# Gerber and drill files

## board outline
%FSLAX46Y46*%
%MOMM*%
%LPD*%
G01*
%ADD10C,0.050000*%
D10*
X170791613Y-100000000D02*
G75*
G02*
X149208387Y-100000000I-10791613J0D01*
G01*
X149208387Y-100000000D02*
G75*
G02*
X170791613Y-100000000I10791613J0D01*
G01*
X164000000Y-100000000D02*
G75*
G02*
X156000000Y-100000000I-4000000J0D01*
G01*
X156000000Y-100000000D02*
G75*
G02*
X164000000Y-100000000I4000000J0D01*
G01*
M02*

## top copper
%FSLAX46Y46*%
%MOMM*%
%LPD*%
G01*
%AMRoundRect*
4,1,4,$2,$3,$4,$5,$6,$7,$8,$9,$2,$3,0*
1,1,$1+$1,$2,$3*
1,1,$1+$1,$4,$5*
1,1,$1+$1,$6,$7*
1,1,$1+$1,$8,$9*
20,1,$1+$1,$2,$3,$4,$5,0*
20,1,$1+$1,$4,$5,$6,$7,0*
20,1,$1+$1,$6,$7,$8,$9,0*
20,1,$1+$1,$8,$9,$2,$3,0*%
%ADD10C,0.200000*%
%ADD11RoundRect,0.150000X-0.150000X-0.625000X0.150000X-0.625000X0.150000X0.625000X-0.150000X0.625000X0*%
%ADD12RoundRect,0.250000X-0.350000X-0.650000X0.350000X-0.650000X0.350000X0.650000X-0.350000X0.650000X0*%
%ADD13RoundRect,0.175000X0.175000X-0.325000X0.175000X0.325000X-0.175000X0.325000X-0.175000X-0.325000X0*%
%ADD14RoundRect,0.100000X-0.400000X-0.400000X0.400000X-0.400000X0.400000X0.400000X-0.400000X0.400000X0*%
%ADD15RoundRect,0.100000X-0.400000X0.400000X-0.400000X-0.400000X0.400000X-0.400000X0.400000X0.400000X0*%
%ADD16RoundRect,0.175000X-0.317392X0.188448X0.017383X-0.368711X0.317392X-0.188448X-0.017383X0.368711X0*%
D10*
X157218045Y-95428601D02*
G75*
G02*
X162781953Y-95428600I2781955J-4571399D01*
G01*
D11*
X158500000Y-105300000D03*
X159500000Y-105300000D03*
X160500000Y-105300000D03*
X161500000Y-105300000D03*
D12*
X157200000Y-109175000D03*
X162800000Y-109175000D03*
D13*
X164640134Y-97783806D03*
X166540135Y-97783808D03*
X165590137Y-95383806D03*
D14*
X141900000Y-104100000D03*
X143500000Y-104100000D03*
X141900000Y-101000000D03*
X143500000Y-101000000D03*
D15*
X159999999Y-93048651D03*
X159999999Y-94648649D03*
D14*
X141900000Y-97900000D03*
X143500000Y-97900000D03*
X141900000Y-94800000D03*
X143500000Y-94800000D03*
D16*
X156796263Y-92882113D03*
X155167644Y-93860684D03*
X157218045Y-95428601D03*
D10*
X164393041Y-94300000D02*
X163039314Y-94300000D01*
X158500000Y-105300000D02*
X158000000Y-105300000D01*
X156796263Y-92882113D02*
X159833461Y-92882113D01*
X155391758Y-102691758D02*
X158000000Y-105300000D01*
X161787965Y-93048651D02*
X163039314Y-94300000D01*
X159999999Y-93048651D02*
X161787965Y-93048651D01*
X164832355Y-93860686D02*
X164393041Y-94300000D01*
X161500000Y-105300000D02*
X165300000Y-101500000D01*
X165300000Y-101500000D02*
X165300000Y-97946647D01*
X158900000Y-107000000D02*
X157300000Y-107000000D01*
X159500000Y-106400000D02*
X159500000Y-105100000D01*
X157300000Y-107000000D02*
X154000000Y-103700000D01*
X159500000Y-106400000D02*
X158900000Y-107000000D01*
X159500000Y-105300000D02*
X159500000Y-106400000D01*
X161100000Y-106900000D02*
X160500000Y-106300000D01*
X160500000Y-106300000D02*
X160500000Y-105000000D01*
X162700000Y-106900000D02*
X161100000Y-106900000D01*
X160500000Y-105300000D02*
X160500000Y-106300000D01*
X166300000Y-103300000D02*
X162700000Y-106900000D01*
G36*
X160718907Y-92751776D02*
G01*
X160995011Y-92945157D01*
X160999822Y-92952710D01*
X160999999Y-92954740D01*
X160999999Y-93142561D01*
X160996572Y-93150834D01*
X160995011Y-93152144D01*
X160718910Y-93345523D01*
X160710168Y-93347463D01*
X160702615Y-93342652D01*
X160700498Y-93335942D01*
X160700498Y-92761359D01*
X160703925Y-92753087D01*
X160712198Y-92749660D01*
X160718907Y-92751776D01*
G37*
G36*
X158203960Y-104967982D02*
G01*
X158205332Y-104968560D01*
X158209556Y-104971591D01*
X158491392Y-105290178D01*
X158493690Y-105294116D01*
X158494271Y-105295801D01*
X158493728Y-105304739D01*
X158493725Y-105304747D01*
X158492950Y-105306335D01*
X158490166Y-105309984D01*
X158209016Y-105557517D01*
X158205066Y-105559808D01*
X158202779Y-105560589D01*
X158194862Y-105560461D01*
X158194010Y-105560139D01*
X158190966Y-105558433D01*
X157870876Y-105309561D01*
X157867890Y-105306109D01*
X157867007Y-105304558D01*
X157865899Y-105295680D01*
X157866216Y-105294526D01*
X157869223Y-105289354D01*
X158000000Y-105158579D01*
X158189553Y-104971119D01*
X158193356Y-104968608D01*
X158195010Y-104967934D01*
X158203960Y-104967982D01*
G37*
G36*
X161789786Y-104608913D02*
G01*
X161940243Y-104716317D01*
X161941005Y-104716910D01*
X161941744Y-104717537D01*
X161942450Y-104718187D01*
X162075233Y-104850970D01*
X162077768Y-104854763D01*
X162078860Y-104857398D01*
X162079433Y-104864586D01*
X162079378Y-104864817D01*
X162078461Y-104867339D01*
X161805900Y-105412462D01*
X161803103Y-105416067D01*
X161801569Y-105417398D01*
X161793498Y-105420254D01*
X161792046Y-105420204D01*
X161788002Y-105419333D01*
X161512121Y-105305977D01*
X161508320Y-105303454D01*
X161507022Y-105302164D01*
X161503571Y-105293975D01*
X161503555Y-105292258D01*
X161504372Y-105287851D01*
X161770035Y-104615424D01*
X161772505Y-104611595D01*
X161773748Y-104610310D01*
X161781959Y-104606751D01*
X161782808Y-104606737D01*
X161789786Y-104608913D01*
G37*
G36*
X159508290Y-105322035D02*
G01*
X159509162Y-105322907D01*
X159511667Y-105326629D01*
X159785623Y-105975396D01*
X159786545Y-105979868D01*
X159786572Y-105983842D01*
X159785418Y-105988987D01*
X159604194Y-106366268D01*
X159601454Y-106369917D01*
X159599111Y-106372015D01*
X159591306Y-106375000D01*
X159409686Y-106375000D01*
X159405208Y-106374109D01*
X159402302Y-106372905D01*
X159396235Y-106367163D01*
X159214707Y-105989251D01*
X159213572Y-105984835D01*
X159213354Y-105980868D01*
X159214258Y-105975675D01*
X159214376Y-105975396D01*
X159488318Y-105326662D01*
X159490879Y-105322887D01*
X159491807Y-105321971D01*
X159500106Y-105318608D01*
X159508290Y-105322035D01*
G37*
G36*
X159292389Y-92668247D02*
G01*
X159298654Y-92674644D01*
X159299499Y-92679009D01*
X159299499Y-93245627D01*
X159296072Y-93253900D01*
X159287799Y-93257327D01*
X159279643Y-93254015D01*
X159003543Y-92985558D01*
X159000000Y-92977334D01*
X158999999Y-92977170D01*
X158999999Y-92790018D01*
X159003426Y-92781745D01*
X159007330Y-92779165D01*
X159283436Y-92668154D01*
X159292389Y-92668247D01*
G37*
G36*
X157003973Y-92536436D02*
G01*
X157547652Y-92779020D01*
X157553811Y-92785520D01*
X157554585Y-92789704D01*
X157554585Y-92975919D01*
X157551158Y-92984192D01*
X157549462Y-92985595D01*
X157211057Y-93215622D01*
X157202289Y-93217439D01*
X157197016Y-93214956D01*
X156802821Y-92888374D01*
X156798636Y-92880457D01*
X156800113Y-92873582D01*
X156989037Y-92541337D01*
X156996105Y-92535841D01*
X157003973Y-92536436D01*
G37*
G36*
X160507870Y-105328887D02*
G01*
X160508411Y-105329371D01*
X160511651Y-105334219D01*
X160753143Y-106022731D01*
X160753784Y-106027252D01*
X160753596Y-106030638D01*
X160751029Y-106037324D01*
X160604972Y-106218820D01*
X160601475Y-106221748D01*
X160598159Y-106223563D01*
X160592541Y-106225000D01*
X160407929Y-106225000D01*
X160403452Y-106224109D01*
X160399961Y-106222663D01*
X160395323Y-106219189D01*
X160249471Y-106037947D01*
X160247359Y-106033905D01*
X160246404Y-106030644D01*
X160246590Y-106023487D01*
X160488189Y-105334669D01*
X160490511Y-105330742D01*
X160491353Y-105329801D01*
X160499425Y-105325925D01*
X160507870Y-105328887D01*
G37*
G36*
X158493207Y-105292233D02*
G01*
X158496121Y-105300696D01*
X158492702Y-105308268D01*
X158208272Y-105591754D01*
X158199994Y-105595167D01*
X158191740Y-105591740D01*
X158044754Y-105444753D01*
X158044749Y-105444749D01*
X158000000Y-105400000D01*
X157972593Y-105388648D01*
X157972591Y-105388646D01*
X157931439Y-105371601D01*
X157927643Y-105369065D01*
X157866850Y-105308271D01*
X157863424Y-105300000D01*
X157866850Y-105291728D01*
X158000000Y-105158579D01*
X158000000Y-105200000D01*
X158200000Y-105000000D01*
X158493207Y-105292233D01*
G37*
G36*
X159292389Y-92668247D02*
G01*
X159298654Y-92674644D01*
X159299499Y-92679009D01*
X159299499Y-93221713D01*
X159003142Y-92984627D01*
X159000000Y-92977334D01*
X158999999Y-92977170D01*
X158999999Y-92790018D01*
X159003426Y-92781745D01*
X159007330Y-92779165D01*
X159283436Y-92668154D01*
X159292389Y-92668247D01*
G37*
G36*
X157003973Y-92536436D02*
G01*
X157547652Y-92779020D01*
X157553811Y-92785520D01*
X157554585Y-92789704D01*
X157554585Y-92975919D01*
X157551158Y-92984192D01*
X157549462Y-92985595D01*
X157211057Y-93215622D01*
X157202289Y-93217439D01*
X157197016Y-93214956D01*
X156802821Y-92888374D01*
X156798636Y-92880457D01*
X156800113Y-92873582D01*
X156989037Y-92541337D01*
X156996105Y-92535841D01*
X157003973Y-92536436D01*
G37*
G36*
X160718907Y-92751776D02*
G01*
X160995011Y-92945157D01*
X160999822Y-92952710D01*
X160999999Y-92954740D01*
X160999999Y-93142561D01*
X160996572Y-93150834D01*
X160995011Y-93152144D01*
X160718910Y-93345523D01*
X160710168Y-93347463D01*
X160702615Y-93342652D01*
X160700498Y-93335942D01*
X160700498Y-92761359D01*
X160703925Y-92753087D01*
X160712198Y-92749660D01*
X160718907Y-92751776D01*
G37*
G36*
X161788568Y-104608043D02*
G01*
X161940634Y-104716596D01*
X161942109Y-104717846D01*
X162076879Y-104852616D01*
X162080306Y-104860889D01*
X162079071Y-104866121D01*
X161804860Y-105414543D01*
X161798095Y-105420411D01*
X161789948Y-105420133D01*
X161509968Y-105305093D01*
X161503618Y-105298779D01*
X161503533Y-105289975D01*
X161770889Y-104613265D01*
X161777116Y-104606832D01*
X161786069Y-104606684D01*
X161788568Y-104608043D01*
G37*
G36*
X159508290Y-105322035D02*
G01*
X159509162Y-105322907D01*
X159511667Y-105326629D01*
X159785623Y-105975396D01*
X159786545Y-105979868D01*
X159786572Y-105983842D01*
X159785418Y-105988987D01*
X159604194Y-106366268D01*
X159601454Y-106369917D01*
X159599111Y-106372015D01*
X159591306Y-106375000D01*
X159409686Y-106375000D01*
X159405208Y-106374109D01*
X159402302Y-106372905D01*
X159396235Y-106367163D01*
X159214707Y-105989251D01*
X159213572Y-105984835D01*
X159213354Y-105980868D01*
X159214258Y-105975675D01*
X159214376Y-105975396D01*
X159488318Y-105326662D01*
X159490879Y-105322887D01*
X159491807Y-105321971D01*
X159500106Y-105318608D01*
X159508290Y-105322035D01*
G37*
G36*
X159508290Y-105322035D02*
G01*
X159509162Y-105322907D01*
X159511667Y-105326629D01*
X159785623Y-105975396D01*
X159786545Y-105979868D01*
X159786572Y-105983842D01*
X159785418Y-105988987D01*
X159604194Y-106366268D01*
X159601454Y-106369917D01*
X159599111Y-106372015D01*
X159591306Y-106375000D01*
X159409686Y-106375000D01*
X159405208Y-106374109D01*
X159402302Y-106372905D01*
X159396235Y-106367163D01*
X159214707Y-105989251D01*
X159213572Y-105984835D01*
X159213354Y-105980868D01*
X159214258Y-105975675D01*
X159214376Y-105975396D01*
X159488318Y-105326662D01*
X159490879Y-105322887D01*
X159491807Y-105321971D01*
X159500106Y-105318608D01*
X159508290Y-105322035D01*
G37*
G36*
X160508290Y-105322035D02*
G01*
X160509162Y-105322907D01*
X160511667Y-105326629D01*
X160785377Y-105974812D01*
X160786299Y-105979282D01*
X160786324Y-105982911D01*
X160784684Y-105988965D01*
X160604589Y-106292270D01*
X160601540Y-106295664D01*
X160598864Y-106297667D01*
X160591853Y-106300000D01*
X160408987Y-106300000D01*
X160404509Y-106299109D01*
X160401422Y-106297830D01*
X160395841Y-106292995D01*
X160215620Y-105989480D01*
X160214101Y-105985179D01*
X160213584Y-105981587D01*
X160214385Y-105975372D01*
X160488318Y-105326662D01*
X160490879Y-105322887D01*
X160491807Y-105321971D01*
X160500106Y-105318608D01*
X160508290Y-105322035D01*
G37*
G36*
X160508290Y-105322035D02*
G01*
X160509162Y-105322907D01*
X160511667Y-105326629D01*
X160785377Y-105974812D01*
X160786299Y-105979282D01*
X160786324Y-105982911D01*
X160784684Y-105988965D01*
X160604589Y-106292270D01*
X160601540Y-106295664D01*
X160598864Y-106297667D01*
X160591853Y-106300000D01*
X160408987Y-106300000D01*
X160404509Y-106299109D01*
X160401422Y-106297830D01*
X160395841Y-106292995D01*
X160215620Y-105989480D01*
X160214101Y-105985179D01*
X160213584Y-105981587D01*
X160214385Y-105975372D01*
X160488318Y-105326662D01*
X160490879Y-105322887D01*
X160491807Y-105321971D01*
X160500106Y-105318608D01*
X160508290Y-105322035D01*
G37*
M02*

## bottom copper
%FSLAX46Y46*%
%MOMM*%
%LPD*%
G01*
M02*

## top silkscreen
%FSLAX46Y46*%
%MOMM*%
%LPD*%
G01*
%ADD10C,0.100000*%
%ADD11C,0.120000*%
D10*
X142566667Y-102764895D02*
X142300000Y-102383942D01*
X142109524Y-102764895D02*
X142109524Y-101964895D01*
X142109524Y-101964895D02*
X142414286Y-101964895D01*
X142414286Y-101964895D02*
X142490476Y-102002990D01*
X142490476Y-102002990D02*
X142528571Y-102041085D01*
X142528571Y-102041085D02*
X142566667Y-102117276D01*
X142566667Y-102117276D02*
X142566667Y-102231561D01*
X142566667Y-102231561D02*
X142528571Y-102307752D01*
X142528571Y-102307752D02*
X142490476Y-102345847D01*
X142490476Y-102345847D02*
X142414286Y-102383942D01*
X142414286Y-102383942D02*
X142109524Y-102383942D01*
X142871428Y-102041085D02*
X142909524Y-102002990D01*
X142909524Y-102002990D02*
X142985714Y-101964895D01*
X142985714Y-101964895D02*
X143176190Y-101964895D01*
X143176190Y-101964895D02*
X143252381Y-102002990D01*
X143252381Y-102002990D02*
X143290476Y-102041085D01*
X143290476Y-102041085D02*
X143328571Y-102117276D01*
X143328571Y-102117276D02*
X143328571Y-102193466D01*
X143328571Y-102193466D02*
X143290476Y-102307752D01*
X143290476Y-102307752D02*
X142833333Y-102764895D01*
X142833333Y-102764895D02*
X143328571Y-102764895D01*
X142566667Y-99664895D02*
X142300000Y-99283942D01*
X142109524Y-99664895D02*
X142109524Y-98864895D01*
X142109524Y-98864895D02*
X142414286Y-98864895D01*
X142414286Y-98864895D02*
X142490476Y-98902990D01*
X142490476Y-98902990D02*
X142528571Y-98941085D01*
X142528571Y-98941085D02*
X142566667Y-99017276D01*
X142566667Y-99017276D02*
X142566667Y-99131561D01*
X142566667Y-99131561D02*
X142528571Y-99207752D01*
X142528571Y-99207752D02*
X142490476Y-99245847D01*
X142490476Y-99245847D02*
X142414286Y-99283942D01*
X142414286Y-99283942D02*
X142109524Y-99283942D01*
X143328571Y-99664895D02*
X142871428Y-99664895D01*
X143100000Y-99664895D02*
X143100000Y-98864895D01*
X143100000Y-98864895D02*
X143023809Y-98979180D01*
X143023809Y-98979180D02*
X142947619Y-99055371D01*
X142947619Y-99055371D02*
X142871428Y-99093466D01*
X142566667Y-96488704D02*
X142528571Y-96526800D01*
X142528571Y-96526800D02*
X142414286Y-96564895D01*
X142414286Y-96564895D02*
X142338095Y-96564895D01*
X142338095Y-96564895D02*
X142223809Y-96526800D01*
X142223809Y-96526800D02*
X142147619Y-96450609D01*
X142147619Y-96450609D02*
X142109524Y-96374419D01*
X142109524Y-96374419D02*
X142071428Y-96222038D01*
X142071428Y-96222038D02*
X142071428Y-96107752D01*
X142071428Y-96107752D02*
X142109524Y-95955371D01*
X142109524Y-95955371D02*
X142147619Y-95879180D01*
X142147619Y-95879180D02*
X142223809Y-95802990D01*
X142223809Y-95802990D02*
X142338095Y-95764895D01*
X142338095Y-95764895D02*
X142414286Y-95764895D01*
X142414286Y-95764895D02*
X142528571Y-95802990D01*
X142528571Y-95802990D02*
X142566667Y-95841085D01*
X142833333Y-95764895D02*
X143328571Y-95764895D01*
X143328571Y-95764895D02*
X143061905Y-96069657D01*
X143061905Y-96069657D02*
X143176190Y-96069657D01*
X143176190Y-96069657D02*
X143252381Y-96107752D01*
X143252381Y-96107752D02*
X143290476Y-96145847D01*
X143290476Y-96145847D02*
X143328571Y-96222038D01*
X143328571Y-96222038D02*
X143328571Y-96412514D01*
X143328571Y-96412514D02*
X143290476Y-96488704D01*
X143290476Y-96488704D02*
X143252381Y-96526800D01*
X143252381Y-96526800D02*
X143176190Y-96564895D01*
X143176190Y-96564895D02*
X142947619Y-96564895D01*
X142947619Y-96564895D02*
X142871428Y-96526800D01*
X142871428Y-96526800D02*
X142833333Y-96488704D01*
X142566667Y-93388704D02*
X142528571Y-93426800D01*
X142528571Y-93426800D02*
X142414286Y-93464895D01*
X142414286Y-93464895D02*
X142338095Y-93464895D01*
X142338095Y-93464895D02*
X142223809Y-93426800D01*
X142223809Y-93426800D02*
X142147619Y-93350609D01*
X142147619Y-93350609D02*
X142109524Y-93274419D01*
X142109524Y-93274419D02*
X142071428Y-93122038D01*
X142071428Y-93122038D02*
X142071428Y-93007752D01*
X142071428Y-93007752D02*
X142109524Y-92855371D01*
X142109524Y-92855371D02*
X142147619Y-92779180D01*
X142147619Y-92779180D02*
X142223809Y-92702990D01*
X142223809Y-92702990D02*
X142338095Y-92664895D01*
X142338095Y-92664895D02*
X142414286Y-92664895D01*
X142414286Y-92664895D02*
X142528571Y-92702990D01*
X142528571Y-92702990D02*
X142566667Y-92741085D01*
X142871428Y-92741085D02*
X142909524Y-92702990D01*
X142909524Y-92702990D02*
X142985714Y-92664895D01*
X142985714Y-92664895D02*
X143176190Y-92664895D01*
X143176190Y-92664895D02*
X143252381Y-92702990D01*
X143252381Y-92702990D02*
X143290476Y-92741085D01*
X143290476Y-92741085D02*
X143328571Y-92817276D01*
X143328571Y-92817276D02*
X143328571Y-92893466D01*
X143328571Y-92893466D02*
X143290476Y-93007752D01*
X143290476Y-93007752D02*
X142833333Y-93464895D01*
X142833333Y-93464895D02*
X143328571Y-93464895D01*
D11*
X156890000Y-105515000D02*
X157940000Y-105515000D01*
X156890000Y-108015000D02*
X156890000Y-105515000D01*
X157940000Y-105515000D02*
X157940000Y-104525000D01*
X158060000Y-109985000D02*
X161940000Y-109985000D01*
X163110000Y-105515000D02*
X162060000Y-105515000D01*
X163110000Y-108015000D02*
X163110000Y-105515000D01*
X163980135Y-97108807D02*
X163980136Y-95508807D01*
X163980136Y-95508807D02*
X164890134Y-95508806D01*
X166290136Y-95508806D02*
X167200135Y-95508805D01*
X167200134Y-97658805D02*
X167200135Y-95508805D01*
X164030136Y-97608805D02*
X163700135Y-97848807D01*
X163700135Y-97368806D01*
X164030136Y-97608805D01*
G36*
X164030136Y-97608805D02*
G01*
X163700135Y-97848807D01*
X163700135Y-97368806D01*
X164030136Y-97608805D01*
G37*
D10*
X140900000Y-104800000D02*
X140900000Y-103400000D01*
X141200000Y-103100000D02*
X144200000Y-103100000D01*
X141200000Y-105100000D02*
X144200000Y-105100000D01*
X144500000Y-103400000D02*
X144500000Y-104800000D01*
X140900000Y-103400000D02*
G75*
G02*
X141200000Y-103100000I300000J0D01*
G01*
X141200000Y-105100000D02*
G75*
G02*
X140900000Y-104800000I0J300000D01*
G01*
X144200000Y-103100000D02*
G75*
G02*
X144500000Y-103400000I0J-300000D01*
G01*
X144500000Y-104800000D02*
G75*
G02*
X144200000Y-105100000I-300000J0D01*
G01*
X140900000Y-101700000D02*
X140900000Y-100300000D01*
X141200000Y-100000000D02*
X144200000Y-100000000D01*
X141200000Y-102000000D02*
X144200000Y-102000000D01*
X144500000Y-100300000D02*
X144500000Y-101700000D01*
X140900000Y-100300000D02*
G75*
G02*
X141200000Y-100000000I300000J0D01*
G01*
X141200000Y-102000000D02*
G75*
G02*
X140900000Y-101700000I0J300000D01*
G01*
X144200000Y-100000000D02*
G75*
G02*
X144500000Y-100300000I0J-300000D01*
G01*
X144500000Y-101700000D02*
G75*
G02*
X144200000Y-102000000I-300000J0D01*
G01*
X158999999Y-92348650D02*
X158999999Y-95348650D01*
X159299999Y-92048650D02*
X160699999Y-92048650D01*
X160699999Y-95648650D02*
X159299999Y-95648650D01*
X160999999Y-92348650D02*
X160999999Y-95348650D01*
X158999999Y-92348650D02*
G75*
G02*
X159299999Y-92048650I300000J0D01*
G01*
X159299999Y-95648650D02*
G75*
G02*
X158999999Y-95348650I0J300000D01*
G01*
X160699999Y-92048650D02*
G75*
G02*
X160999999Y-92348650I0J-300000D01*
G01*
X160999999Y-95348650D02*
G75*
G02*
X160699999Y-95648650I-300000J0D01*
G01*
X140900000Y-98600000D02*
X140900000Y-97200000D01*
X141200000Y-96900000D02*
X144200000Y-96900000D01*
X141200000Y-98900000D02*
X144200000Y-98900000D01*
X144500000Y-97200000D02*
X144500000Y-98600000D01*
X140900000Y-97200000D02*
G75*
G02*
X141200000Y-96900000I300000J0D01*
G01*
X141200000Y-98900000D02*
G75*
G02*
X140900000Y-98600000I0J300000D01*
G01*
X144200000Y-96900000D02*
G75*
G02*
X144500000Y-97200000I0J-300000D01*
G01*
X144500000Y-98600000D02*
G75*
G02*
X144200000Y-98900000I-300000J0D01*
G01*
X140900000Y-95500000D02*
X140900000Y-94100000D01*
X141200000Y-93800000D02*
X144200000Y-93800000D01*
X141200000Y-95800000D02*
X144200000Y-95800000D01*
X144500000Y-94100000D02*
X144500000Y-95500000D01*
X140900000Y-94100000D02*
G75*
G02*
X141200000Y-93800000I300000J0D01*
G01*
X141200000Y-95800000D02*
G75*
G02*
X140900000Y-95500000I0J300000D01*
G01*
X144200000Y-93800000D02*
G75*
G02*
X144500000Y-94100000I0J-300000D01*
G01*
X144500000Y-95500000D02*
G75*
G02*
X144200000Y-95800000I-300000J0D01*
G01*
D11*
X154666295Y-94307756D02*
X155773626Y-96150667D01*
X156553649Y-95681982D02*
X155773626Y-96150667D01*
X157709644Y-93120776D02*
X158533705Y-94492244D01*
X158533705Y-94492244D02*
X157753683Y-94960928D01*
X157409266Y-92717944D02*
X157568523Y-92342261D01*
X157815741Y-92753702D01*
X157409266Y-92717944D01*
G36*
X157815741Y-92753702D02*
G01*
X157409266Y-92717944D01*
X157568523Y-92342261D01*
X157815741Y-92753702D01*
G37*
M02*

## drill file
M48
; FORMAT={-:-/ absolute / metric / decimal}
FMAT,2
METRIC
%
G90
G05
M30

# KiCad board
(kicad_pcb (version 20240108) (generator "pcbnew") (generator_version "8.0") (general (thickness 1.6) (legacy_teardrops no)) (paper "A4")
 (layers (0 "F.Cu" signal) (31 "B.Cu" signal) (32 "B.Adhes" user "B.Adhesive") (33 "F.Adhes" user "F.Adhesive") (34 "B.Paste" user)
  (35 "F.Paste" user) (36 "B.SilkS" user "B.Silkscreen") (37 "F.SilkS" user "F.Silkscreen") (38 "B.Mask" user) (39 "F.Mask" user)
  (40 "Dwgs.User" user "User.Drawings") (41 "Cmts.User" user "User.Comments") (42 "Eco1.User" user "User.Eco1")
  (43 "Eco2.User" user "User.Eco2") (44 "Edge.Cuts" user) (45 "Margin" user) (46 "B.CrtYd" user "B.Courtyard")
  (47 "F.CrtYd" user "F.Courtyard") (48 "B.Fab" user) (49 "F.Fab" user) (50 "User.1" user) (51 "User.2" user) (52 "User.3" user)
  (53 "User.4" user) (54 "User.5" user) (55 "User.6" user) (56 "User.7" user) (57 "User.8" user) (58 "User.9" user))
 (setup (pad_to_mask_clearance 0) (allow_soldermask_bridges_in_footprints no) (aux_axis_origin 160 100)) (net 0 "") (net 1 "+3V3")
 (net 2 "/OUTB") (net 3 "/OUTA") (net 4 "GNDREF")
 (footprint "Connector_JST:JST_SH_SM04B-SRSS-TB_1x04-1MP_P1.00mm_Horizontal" (layer "F.Cu") (at 160 107.3)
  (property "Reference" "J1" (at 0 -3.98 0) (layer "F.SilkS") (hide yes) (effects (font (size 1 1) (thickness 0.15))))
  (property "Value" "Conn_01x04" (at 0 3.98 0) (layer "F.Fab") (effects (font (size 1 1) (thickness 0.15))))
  (fp_line (start -3.11 -1.785) (end -2.06 -1.785) (stroke (width 0.12) (type solid)) (layer "F.SilkS"))
  (fp_line (start -3.11 0.715) (end -3.11 -1.785) (stroke (width 0.12) (type solid)) (layer "F.SilkS"))
  (fp_line (start -2.06 -1.785) (end -2.06 -2.775) (stroke (width 0.12) (type solid)) (layer "F.SilkS"))
  (fp_line (start -1.94 2.685) (end 1.94 2.685) (stroke (width 0.12) (type solid)) (layer "F.SilkS"))
  (fp_line (start 3.11 -1.785) (end 2.06 -1.785) (stroke (width 0.12) (type solid)) (layer "F.SilkS"))
  (fp_line (start 3.11 0.715) (end 3.11 -1.785) (stroke (width 0.12) (type solid)) (layer "F.SilkS"))
  (pad "1" smd roundrect (at -1.5 -2) (size 0.6 1.55) (layers "F.Cu" "F.Paste" "F.Mask") (roundrect_rratio 0.25) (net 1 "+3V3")
   (teardrops (best_length_ratio 0.5) (max_length 1) (best_width_ratio 1) (max_width 2) (curve_points 0) (filter_ratio 0.9) (enabled yes)
    (allow_two_segments yes) (prefer_zone_connections yes)))
  (pad "2" smd roundrect (at -0.5 -2) (size 0.6 1.55) (layers "F.Cu" "F.Paste" "F.Mask") (roundrect_rratio 0.25) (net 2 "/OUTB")
   (teardrops (best_length_ratio 0.5) (max_length 1) (best_width_ratio 1) (max_width 2) (curve_points 0) (filter_ratio 0.9) (enabled yes)
    (allow_two_segments yes) (prefer_zone_connections yes)))
  (pad "3" smd roundrect (at 0.5 -2) (size 0.6 1.55) (layers "F.Cu" "F.Paste" "F.Mask") (roundrect_rratio 0.25) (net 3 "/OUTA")
   (teardrops (best_length_ratio 0.5) (max_length 1) (best_width_ratio 1) (max_width 2) (curve_points 0) (filter_ratio 0.9) (enabled yes)
    (allow_two_segments yes) (prefer_zone_connections yes)))
  (pad "4" smd roundrect (at 1.5 -2) (size 0.6 1.55) (layers "F.Cu" "F.Paste" "F.Mask") (roundrect_rratio 0.25) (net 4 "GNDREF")
   (teardrops (best_length_ratio 0.5) (max_length 1) (best_width_ratio 1) (max_width 2) (curve_points 0) (filter_ratio 0.9) (enabled yes)
    (allow_two_segments yes) (prefer_zone_connections yes)))
  (pad "MP" smd roundrect (at -2.8 1.875) (size 1.2 1.8) (layers "F.Cu" "F.Paste" "F.Mask") (roundrect_rratio 0.208333)
   (teardrops (best_length_ratio 0.5) (max_length 1) (best_width_ratio 1) (max_width 2) (curve_points 0) (filter_ratio 0.9) (enabled yes)
    (allow_two_segments yes) (prefer_zone_connections yes)))
  (pad "MP" smd roundrect (at 2.8 1.875) (size 1.2 1.8) (layers "F.Cu" "F.Paste" "F.Mask") (roundrect_rratio 0.208333)
   (teardrops (best_length_ratio 0.5) (max_length 1) (best_width_ratio 1) (max_width 2) (curve_points 0) (filter_ratio 0.9) (enabled yes)
    (allow_two_segments yes) (prefer_zone_connections yes))))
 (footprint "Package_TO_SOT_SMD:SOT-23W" (layer "F.Cu") (at 165.590135 96.583806 90)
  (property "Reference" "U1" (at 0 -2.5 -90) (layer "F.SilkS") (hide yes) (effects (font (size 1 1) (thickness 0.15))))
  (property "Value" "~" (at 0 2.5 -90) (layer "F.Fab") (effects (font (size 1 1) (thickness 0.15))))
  (fp_line (start -0.525001 -1.61) (end 1.074999 -1.609999) (stroke (width 0.12) (type solid)) (layer "F.SilkS"))
  (fp_line (start 1.074999 -1.609999) (end 1.075 -0.700001) (stroke (width 0.12) (type solid)) (layer "F.SilkS"))
  (fp_line (start 1.075 0.700001) (end 1.075001 1.61) (stroke (width 0.12) (type solid)) (layer "F.SilkS"))
  (fp_line (start -1.074999 1.609999) (end 1.075001 1.61) (stroke (width 0.12) (type solid)) (layer "F.SilkS"))
  (fp_poly
   (pts (xy -1.024999 -1.559999) (xy -1.265001 -1.89) (xy -0.785 -1.89) (xy -1.024999 -1.559999)) (stroke (width 0.12) (type solid))
   (fill solid) (layer "F.SilkS"))
  (pad "1" smd roundrect (at -1.2 -0.950001 90) (size 1 0.7) (layers "F.Cu" "F.Paste" "F.Mask") (roundrect_rratio 0.25) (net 1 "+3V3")
   (teardrops (best_length_ratio 0.5) (max_length 1) (best_width_ratio 1) (max_width 2) (curve_points 0) (filter_ratio 0.9) (enabled yes)
    (allow_two_segments yes) (prefer_zone_connections yes)))
  (pad "2" smd roundrect (at -1.200002 0.95 90) (size 1 0.7) (layers "F.Cu" "F.Paste" "F.Mask") (roundrect_rratio 0.25) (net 3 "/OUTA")
   (teardrops (best_length_ratio 0.5) (max_length 1) (best_width_ratio 1) (max_width 2) (curve_points 0) (filter_ratio 0.9) (enabled yes)
    (allow_two_segments yes) (prefer_zone_connections yes)))
  (pad "3" smd roundrect (at 1.2 0.000002 90) (size 1 0.7) (layers "F.Cu" "F.Paste" "F.Mask") (roundrect_rratio 0.25) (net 4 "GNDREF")
   (teardrops (best_length_ratio 0.5) (max_length 1) (best_width_ratio 1) (max_width 2) (curve_points 0) (filter_ratio 0.9) (enabled yes)
    (allow_two_segments yes) (prefer_zone_connections yes))))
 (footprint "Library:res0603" (layer "F.Cu") (at 142.7 104.1)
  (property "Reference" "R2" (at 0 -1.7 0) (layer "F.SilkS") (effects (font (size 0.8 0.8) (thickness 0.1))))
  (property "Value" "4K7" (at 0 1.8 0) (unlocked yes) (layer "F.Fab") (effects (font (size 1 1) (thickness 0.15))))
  (fp_line (start -1.8 0.7) (end -1.8 -0.7) (stroke (width 0.1) (type default)) (layer "F.SilkS"))
  (fp_line (start -1.5 -1) (end 1.5 -1) (stroke (width 0.1) (type default)) (layer "F.SilkS"))
  (fp_line (start -1.5 1) (end 1.5 1) (stroke (width 0.1) (type default)) (layer "F.SilkS"))
  (fp_line (start 1.8 -0.7) (end 1.8 0.7) (stroke (width 0.1) (type default)) (layer "F.SilkS"))
  (fp_arc (start -1.8 -0.7) (mid -1.712132 -0.912132) (end -1.5 -1) (stroke (width 0.1) (type default)) (layer "F.SilkS"))
  (fp_arc (start -1.5 1) (mid -1.712132 0.912132) (end -1.8 0.7) (stroke (width 0.1) (type default)) (layer "F.SilkS"))
  (fp_arc (start 1.5 -1) (mid 1.712132 -0.912132) (end 1.8 -0.7) (stroke (width 0.1) (type default)) (layer "F.SilkS"))
  (fp_arc (start 1.8 0.7) (mid 1.712132 0.912132) (end 1.5 1) (stroke (width 0.1) (type default)) (layer "F.SilkS"))
  (pad "1" smd roundrect (at -0.8 0) (size 1 1) (layers "F.Cu" "F.Paste" "F.Mask") (roundrect_rratio 0.1) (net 2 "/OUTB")
   (thermal_bridge_angle 45)
   (teardrops (best_length_ratio 0.5) (max_length 1) (best_width_ratio 1) (max_width 1) (curve_points 10) (filter_ratio 0.9) (enabled yes)
    (allow_two_segments yes) (prefer_zone_connections yes)))
  (pad "2" smd roundrect (at 0.8 0) (size 1 1) (layers "F.Cu" "F.Paste" "F.Mask") (roundrect_rratio 0.1) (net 4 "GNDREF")
   (thermal_bridge_angle 45)
   (teardrops (best_length_ratio 0.5) (max_length 1) (best_width_ratio 1) (max_width 1) (curve_points 10) (filter_ratio 0.9) (enabled yes)
    (allow_two_segments yes) (prefer_zone_connections yes))))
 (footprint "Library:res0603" (layer "F.Cu") (at 142.7 101)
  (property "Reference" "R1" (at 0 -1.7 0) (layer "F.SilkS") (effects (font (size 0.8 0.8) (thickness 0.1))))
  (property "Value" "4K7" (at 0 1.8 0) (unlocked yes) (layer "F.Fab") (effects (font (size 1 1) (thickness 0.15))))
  (fp_line (start -1.8 0.7) (end -1.8 -0.7) (stroke (width 0.1) (type default)) (layer "F.SilkS"))
  (fp_line (start -1.5 -1) (end 1.5 -1) (stroke (width 0.1) (type default)) (layer "F.SilkS"))
  (fp_line (start -1.5 1) (end 1.5 1) (stroke (width 0.1) (type default)) (layer "F.SilkS"))
  (fp_line (start 1.8 -0.7) (end 1.8 0.7) (stroke (width 0.1) (type default)) (layer "F.SilkS"))
  (fp_arc (start -1.8 -0.7) (mid -1.712132 -0.912132) (end -1.5 -1) (stroke (width 0.1) (type default)) (layer "F.SilkS"))
  (fp_arc (start -1.5 1) (mid -1.712132 0.912132) (end -1.8 0.7) (stroke (width 0.1) (type default)) (layer "F.SilkS"))
  (fp_arc (start 1.5 -1) (mid 1.712132 -0.912132) (end 1.8 -0.7) (stroke (width 0.1) (type default)) (layer "F.SilkS"))
  (fp_arc (start 1.8 0.7) (mid 1.712132 0.912132) (end 1.5 1) (stroke (width 0.1) (type default)) (layer "F.SilkS"))
  (pad "1" smd roundrect (at -0.8 0) (size 1 1) (layers "F.Cu" "F.Paste" "F.Mask") (roundrect_rratio 0.1) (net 3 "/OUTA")
   (thermal_bridge_angle 45)
   (teardrops (best_length_ratio 0.5) (max_length 1) (best_width_ratio 1) (max_width 1) (curve_points 10) (filter_ratio 0.9) (enabled yes)
    (allow_two_segments yes) (prefer_zone_connections yes)))
  (pad "2" smd roundrect (at 0.8 0) (size 1 1) (layers "F.Cu" "F.Paste" "F.Mask") (roundrect_rratio 0.1) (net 4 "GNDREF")
   (thermal_bridge_angle 45)
   (teardrops (best_length_ratio 0.5) (max_length 1) (best_width_ratio 1) (max_width 1) (curve_points 10) (filter_ratio 0.9) (enabled yes)
    (allow_two_segments yes) (prefer_zone_connections yes))))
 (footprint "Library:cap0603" (layer "F.Cu") (at 159.999999 93.84865 -90)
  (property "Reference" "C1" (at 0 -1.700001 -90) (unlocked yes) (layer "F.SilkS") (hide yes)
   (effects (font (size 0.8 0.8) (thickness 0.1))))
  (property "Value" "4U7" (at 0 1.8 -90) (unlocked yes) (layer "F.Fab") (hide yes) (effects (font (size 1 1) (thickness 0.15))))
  (fp_line (start -1.5 1) (end 1.5 1) (stroke (width 0.1) (type default)) (layer "F.SilkS"))
  (fp_line (start -1.8 0.7) (end -1.8 -0.7) (stroke (width 0.1) (type default)) (layer "F.SilkS"))
  (fp_line (start 1.8 -0.7) (end 1.8 0.7) (stroke (width 0.1) (type default)) (layer "F.SilkS"))
  (fp_line (start -1.5 -1) (end 1.5 -1) (stroke (width 0.1) (type default)) (layer "F.SilkS"))
  (fp_arc (start -1.5 1) (mid -1.712132 0.912132) (end -1.8 0.7) (stroke (width 0.1) (type default)) (layer "F.SilkS"))
  (fp_arc (start 1.8 0.7) (mid 1.712132 0.912132) (end 1.5 1) (stroke (width 0.1) (type default)) (layer "F.SilkS"))
  (fp_arc (start -1.8 -0.7) (mid -1.712132 -0.912132) (end -1.5 -1) (stroke (width 0.1) (type default)) (layer "F.SilkS"))
  (fp_arc (start 1.5 -1) (mid 1.712132 -0.912132) (end 1.8 -0.7) (stroke (width 0.1) (type default)) (layer "F.SilkS"))
  (pad "1" smd roundrect (at -0.799999 0 270) (size 1 1) (layers "F.Cu" "F.Paste" "F.Mask") (roundrect_rratio 0.1) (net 3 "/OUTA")
   (thermal_bridge_angle 45)
   (teardrops (best_length_ratio 0.5) (max_length 1) (best_width_ratio 1) (max_width 2) (curve_points 0) (filter_ratio 0.9) (enabled yes)
    (allow_two_segments yes) (prefer_zone_connections yes)))
  (pad "2" smd roundrect (at 0.799999 0 270) (size 1 1) (layers "F.Cu" "F.Paste" "F.Mask") (roundrect_rratio 0.1) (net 4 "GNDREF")
   (thermal_bridge_angle 45)
   (teardrops (best_length_ratio 0.5) (max_length 1) (best_width_ratio 1) (max_width 2) (curve_points 0) (filter_ratio 0.9) (enabled yes)
    (allow_two_segments yes) (prefer_zone_connections yes))))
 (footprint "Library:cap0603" (layer "F.Cu") (at 142.7 97.9)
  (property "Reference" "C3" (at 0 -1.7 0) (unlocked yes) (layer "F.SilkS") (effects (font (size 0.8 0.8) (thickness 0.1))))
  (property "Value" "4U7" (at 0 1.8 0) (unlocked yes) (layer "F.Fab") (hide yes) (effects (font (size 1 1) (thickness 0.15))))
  (fp_line (start -1.8 0.7) (end -1.8 -0.7) (stroke (width 0.1) (type default)) (layer "F.SilkS"))
  (fp_line (start -1.5 -1) (end 1.5 -1) (stroke (width 0.1) (type default)) (layer "F.SilkS"))
  (fp_line (start -1.5 1) (end 1.5 1) (stroke (width 0.1) (type default)) (layer "F.SilkS"))
  (fp_line (start 1.8 -0.7) (end 1.8 0.7) (stroke (width 0.1) (type default)) (layer "F.SilkS"))
  (fp_arc (start -1.8 -0.7) (mid -1.712132 -0.912132) (end -1.5 -1) (stroke (width 0.1) (type default)) (layer "F.SilkS"))
  (fp_arc (start -1.5 1) (mid -1.712132 0.912132) (end -1.8 0.7) (stroke (width 0.1) (type default)) (layer "F.SilkS"))
  (fp_arc (start 1.5 -1) (mid 1.712132 -0.912132) (end 1.8 -0.7) (stroke (width 0.1) (type default)) (layer "F.SilkS"))
  (fp_arc (start 1.8 0.7) (mid 1.712132 0.912132) (end 1.5 1) (stroke (width 0.1) (type default)) (layer "F.SilkS"))
  (pad "1" smd roundrect (at -0.8 0) (size 1 1) (layers "F.Cu" "F.Paste" "F.Mask") (roundrect_rratio 0.1) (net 2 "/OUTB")
   (thermal_bridge_angle 45)
   (teardrops (best_length_ratio 0.5) (max_length 1) (best_width_ratio 1) (max_width 1) (curve_points 10) (filter_ratio 0.9) (enabled yes)
    (allow_two_segments yes) (prefer_zone_connections yes)))
  (pad "2" smd roundrect (at 0.8 0) (size 1 1) (layers "F.Cu" "F.Paste" "F.Mask") (roundrect_rratio 0.1) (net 4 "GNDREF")
   (thermal_bridge_angle 45)
   (teardrops (best_length_ratio 0.5) (max_length 1) (best_width_ratio 1) (max_width 1) (curve_points 10) (filter_ratio 0.9) (enabled yes)
    (allow_two_segments yes) (prefer_zone_connections yes))))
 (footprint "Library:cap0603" (layer "F.Cu") (at 142.7 94.8)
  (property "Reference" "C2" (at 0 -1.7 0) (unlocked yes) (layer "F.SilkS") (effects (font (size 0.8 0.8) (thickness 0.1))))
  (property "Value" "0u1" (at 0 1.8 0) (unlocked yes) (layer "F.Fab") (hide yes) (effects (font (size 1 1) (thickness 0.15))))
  (fp_line (start -1.8 0.7) (end -1.8 -0.7) (stroke (width 0.1) (type default)) (layer "F.SilkS"))
  (fp_line (start -1.5 -1) (end 1.5 -1) (stroke (width 0.1) (type default)) (layer "F.SilkS"))
  (fp_line (start -1.5 1) (end 1.5 1) (stroke (width 0.1) (type default)) (layer "F.SilkS"))
  (fp_line (start 1.8 -0.7) (end 1.8 0.7) (stroke (width 0.1) (type default)) (layer "F.SilkS"))
  (fp_arc (start -1.8 -0.7) (mid -1.712132 -0.912132) (end -1.5 -1) (stroke (width 0.1) (type default)) (layer "F.SilkS"))
  (fp_arc (start -1.5 1) (mid -1.712132 0.912132) (end -1.8 0.7) (stroke (width 0.1) (type default)) (layer "F.SilkS"))
  (fp_arc (start 1.5 -1) (mid 1.712132 -0.912132) (end 1.8 -0.7) (stroke (width 0.1) (type default)) (layer "F.SilkS"))
  (fp_arc (start 1.8 0.7) (mid 1.712132 0.912132) (end 1.5 1) (stroke (width 0.1) (type default)) (layer "F.SilkS"))
  (pad "1" smd roundrect (at -0.8 0) (size 1 1) (layers "F.Cu" "F.Paste" "F.Mask") (roundrect_rratio 0.1) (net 1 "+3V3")
   (thermal_bridge_angle 45)
   (teardrops (best_length_ratio 0.5) (max_length 1) (best_width_ratio 1) (max_width 1) (curve_points 10) (filter_ratio 0.9) (enabled yes)
    (allow_two_segments yes) (prefer_zone_connections yes)))
  (pad "2" smd roundrect (at 0.8 0) (size 1 1) (layers "F.Cu" "F.Paste" "F.Mask") (roundrect_rratio 0.1) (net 4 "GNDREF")
   (thermal_bridge_angle 45)
   (teardrops (best_length_ratio 0.5) (max_length 1) (best_width_ratio 1) (max_width 1) (curve_points 10) (filter_ratio 0.9) (enabled yes)
    (allow_two_segments yes) (prefer_zone_connections yes))))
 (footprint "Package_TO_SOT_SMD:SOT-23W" (layer "F.Cu") (at 156.6 94.4 -59)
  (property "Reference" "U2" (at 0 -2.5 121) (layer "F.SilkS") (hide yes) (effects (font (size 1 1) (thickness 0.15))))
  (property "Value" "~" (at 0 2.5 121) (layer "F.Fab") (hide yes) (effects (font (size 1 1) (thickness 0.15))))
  (fp_line (start -1.075 1.61) (end 1.075 1.610001) (stroke (width 0.12) (type solid)) (layer "F.SilkS"))
  (fp_line (start 1.075001 0.7) (end 1.075 1.610001) (stroke (width 0.12) (type solid)) (layer "F.SilkS"))
  (fp_line (start -0.525 -1.61) (end 1.075 -1.61) (stroke (width 0.12) (type solid)) (layer "F.SilkS"))
  (fp_line (start 1.075 -1.61) (end 1.075 -0.7) (stroke (width 0.12) (type solid)) (layer "F.SilkS"))
  (fp_poly
   (pts (xy -1.025001 -1.559999) (xy -1.265 -1.89) (xy -0.785 -1.89) (xy -1.025001 -1.559999)) (stroke (width 0.12) (type solid))
   (fill solid) (layer "F.SilkS"))
  (pad "1" smd roundrect (at -1.2 -0.95 301) (size 1 0.7) (layers "F.Cu" "F.Paste" "F.Mask") (roundrect_rratio 0.25) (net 1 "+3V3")
   (teardrops (best_length_ratio 0.5) (max_length 1) (best_width_ratio 1) (max_width 2) (curve_points 0) (filter_ratio 0.9) (enabled yes)
    (allow_two_segments yes) (prefer_zone_connections yes)))
  (pad "2" smd roundrect (at -1.200002 0.95 301) (size 1 0.7) (layers "F.Cu" "F.Paste" "F.Mask") (roundrect_rratio 0.25) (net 2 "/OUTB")
   (teardrops (best_length_ratio 0.5) (max_length 1) (best_width_ratio 1) (max_width 2) (curve_points 0) (filter_ratio 0.9) (enabled yes)
    (allow_two_segments yes) (prefer_zone_connections yes)))
  (pad "3" smd roundrect (at 1.2 0.000001 301) (size 1 0.7) (layers "F.Cu" "F.Paste" "F.Mask") (roundrect_rratio 0.25) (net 4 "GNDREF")
   (teardrops (best_length_ratio 0.5) (max_length 1) (best_width_ratio 1) (max_width 2) (curve_points 0) (filter_ratio 0.9) (enabled yes)
    (allow_two_segments yes) (prefer_zone_connections yes))))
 (gr_arc (start 157.218045 95.428601) (mid 159.999999 94.648649) (end 162.781953 95.4286) (stroke (width 0.2) (type default)) (layer "F.Cu")
  (net 4))
 (gr_circle (center 160 100) (end 160 89.208387) (stroke (width 0.05) (type default)) (fill none) (layer "Edge.Cuts"))
 (gr_circle (center 160 100) (end 164 100) (stroke (width 0.05) (type default)) (fill none) (layer "Edge.Cuts"))
 (segment (start 164.393041 94.3) (end 163.039314 94.3) (width 0.2) (layer "F.Cu") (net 1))
 (segment (start 158.5 105.3) (end 158 105.3) (width 0.2) (layer "F.Cu") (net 1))
 (segment (start 156.796263 92.882113) (end 159.833461 92.882113) (width 0.2) (layer "F.Cu") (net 1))
 (segment (start 155.391758 102.691758) (end 158 105.3) (width 0.2) (layer "F.Cu") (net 1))
 (segment (start 161.787965 93.048651) (end 163.039314 94.3) (width 0.2) (layer "F.Cu") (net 1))
 (segment (start 159.999999 93.048651) (end 161.787965 93.048651) (width 0.2) (layer "F.Cu") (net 1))
 (segment (start 164.832355 93.860686) (end 164.393041 94.3) (width 0.2) (layer "F.Cu") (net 1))
 (segment (start 161.5 105.3) (end 165.3 101.5) (width 0.2) (layer "F.Cu") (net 4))
 (segment (start 165.3 101.5) (end 165.3 97.946647) (width 0.2) (layer "F.Cu") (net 4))
 (segment (start 158.9 107) (end 157.3 107) (width 0.2) (layer "F.Cu") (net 2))
 (segment (start 159.5 106.4) (end 159.5 105.1) (width 0.2) (layer "F.Cu") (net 2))
 (segment (start 157.3 107) (end 154 103.7) (width 0.2) (layer "F.Cu") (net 2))
 (segment (start 159.5 106.4) (end 158.9 107) (width 0.2) (layer "F.Cu") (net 2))
 (segment (start 159.5 105.3) (end 159.5 106.4) (width 0.2) (layer "F.Cu") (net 2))
 (segment (start 161.1 106.9) (end 160.5 106.3) (width 0.2) (layer "F.Cu") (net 3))
 (segment (start 160.5 106.3) (end 160.5 105) (width 0.2) (layer "F.Cu") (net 3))
 (segment (start 162.7 106.9) (end 161.1 106.9) (width 0.2) (layer "F.Cu") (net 3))
 (segment (start 160.5 105.3) (end 160.5 106.3) (width 0.2) (layer "F.Cu") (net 3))
 (segment (start 166.3 103.3) (end 162.7 106.9) (width 0.2) (layer "F.Cu") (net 3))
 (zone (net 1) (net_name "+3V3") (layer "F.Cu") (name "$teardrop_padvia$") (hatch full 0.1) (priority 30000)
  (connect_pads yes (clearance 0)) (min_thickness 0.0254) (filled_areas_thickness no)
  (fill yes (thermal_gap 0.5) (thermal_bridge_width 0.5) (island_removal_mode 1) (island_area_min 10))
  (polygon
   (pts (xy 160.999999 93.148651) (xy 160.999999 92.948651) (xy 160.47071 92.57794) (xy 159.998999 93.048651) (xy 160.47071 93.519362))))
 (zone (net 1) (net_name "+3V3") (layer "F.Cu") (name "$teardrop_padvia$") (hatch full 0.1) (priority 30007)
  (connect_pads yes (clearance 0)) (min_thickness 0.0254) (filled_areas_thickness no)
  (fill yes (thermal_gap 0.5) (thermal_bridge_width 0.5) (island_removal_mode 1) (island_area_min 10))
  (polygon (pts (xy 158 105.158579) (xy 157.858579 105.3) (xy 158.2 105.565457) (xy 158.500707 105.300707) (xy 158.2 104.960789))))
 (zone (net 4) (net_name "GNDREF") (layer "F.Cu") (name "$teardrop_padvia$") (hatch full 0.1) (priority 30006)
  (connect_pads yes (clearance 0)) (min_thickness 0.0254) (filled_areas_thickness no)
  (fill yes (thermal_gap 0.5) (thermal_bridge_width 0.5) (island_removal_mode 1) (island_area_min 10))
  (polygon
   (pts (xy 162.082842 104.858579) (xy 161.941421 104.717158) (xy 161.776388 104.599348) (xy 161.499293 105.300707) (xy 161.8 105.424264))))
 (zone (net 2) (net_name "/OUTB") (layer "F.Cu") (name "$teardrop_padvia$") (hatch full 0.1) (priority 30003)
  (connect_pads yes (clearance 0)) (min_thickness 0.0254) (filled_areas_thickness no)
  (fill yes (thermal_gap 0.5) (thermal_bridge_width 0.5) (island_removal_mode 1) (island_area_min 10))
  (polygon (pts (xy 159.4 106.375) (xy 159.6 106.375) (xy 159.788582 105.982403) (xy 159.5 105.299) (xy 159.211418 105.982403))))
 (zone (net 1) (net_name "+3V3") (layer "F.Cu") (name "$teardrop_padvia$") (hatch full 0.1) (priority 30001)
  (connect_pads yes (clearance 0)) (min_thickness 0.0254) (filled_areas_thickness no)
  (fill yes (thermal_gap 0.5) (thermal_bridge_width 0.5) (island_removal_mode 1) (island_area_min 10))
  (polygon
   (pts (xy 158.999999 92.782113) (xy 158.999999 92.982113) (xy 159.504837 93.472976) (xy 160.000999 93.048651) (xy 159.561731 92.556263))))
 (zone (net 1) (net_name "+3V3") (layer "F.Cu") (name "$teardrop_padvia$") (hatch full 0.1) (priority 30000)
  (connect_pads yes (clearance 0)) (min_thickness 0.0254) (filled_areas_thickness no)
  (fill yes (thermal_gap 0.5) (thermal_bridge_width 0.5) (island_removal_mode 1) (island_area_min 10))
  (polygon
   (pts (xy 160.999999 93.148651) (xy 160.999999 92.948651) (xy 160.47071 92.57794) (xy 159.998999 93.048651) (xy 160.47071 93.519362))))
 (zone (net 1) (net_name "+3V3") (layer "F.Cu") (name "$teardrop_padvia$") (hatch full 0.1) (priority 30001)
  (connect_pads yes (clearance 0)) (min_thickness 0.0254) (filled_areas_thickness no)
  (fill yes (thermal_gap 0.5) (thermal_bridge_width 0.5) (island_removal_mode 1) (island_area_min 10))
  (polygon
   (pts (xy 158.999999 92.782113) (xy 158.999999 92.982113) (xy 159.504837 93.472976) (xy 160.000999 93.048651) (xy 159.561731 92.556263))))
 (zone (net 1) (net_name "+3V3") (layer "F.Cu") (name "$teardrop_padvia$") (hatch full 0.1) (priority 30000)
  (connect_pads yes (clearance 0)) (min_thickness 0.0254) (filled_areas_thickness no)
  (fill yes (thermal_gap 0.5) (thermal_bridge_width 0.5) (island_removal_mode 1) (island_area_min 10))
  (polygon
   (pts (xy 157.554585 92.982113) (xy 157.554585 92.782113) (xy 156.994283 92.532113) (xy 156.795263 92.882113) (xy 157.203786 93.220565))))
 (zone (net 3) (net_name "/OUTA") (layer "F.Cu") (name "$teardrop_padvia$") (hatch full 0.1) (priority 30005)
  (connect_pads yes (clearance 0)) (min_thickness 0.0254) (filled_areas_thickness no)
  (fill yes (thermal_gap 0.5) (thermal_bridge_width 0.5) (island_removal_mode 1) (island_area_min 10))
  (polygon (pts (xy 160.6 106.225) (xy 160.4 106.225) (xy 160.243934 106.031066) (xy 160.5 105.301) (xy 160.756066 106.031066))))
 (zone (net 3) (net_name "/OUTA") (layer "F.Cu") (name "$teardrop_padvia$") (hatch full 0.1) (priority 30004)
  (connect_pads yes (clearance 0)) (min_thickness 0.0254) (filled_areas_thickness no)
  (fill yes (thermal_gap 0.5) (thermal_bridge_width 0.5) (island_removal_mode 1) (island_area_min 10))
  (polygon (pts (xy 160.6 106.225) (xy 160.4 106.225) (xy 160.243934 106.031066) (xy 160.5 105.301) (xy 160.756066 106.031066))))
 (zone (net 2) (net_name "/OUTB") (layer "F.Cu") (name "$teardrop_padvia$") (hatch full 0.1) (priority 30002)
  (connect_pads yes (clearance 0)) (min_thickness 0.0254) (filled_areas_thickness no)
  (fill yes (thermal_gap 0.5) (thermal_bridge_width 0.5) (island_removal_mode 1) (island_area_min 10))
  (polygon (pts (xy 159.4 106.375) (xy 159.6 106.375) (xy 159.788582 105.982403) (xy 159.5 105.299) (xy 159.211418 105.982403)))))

